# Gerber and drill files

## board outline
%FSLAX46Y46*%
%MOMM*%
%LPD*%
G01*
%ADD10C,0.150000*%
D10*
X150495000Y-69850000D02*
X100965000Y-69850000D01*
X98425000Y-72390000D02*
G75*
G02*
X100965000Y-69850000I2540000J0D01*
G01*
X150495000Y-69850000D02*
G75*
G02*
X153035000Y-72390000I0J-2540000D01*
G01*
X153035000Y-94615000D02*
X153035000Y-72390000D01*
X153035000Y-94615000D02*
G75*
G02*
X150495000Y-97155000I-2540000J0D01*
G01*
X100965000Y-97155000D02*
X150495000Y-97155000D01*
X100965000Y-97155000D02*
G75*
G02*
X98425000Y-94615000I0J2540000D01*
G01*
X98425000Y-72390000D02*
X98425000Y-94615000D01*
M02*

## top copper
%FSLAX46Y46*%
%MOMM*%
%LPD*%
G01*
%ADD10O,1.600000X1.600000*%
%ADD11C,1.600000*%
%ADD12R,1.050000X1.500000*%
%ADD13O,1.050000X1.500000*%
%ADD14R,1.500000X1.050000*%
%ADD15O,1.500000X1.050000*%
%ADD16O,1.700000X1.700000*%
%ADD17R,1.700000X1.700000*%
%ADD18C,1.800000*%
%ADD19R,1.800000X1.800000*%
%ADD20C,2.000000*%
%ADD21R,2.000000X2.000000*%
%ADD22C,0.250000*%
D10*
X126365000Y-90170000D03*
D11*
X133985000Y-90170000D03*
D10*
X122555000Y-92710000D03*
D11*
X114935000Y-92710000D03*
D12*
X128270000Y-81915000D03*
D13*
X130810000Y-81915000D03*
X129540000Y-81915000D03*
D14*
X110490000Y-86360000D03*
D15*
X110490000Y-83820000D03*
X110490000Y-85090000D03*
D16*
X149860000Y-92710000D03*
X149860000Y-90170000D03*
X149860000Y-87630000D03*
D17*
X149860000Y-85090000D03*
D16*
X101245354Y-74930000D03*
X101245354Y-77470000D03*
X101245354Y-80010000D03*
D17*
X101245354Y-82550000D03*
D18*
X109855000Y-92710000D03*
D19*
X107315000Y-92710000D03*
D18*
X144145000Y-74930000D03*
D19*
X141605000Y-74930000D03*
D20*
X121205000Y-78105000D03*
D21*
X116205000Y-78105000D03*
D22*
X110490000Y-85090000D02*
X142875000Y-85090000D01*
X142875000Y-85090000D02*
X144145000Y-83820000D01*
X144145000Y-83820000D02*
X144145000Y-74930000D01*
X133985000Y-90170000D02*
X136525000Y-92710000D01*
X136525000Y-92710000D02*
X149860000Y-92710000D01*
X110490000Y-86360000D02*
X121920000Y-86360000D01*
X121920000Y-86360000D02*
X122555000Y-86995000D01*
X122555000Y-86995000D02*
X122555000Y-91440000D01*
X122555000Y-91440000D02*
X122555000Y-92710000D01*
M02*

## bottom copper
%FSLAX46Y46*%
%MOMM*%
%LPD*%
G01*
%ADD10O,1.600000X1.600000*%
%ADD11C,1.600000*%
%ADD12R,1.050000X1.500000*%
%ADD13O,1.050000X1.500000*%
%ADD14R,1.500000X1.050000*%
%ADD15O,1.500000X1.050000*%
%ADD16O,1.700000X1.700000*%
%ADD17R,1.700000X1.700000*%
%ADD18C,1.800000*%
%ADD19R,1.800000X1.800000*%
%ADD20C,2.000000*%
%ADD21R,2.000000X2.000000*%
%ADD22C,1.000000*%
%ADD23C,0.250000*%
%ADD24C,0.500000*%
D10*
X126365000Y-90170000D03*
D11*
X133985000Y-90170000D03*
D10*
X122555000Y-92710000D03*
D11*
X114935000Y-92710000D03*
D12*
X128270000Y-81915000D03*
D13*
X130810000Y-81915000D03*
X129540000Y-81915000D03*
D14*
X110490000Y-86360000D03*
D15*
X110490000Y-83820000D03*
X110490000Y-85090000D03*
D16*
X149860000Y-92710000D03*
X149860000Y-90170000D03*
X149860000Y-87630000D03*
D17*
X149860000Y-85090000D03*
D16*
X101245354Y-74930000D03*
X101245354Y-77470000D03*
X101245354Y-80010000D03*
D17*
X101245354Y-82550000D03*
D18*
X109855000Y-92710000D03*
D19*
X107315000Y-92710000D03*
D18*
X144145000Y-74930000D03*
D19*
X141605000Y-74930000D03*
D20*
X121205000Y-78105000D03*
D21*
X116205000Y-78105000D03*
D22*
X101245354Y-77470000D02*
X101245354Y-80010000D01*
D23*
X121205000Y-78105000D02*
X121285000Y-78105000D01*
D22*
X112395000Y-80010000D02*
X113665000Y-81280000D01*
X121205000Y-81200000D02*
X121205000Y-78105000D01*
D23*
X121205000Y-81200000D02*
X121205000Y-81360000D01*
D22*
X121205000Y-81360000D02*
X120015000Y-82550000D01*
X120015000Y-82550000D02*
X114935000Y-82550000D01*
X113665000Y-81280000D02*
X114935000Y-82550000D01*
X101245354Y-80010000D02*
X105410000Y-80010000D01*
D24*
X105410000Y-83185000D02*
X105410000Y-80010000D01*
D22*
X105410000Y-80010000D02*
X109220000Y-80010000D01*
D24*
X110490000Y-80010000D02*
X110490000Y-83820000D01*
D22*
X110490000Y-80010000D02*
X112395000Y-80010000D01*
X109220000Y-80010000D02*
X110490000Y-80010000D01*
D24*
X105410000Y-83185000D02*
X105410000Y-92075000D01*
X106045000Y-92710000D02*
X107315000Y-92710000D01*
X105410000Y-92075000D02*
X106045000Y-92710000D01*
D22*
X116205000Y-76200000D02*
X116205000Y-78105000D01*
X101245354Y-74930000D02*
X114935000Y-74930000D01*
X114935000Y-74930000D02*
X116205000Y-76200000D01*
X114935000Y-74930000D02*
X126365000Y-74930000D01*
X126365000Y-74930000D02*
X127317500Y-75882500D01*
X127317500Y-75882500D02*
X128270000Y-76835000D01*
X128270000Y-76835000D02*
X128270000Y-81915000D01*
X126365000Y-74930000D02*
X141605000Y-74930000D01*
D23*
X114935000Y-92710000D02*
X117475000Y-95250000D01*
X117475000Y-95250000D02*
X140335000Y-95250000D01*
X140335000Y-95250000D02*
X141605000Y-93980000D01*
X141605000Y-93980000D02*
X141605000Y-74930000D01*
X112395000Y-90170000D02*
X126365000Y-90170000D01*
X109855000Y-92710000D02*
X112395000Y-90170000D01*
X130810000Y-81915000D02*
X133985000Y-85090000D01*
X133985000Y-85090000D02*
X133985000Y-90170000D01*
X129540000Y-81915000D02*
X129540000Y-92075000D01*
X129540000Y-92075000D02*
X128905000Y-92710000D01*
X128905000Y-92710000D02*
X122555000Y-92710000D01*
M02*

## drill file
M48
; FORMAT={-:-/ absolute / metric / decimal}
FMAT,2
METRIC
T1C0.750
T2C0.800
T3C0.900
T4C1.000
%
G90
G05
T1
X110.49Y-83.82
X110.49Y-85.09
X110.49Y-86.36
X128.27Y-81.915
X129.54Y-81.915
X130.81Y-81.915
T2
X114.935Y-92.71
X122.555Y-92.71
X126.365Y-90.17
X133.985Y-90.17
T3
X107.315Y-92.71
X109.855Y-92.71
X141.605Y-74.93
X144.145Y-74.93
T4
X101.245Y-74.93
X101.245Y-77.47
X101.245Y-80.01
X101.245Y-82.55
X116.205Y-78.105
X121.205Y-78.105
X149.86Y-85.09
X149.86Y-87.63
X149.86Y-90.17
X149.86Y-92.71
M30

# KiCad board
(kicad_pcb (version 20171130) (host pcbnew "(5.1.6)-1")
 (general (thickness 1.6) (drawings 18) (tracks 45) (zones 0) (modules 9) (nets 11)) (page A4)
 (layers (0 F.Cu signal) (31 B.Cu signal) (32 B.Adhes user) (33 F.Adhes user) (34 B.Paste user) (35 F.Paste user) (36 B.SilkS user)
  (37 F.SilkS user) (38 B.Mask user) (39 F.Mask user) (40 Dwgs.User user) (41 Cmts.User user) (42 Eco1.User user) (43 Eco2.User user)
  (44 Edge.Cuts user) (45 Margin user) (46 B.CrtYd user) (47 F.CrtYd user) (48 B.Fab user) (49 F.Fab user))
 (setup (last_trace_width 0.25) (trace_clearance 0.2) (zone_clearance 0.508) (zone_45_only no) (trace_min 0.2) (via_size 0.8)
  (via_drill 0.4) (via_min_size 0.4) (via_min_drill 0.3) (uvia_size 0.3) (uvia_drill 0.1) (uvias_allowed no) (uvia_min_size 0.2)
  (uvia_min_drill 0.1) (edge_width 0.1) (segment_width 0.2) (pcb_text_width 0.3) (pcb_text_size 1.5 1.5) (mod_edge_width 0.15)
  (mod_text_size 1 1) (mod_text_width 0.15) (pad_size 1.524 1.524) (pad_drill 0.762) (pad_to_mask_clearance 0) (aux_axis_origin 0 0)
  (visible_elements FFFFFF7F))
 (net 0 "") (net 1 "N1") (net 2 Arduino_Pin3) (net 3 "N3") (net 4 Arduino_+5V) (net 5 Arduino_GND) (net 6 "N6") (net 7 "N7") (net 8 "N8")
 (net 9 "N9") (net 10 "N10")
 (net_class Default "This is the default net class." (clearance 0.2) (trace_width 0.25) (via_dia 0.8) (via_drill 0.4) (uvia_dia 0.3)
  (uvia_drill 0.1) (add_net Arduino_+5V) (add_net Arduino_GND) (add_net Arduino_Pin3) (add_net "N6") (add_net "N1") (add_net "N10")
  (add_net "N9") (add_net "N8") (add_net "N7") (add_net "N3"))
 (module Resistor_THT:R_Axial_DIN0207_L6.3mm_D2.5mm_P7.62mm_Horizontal (layer F.Cu) (at 133.985 90.17 180)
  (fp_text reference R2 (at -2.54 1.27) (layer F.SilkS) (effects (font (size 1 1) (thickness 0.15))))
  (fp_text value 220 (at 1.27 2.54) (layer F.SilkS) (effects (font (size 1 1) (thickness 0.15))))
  (pad 2 thru_hole oval (at 7.62 0 180) (size 1.6 1.6) (drill 0.8) (layers *.Cu *.Mask) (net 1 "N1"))
  (pad 1 thru_hole circle (at 0 0 180) (size 1.6 1.6) (drill 0.8) (layers *.Cu *.Mask) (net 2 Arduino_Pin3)))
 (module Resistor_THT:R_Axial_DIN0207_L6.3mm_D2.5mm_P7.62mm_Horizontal (layer F.Cu) (at 114.935 92.71)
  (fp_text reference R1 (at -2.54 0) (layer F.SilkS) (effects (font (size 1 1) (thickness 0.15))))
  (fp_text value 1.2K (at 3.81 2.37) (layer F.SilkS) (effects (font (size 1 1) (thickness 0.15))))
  (pad 2 thru_hole oval (at 7.62 0) (size 1.6 1.6) (drill 0.8) (layers *.Cu *.Mask) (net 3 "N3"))
  (pad 1 thru_hole circle (at 0 0) (size 1.6 1.6) (drill 0.8) (layers *.Cu *.Mask) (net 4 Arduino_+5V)))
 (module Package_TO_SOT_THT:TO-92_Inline (layer F.Cu) (at 128.27 81.915)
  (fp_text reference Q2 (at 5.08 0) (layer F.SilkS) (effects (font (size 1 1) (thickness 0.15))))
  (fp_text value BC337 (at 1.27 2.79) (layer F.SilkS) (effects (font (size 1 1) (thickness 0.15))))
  (pad 1 thru_hole rect (at 0 0) (size 1.05 1.5) (drill 0.75) (layers *.Cu *.Mask) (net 4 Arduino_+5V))
  (pad 3 thru_hole oval (at 2.54 0) (size 1.05 1.5) (drill 0.75) (layers *.Cu *.Mask) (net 2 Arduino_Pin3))
  (pad 2 thru_hole oval (at 1.27 0) (size 1.05 1.5) (drill 0.75) (layers *.Cu *.Mask) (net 3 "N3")))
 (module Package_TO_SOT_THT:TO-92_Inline (layer F.Cu) (at 110.49 86.36 90)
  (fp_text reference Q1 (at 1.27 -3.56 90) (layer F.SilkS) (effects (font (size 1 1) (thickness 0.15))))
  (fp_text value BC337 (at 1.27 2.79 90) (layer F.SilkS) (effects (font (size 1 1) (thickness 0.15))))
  (pad 1 thru_hole rect (at 0 0 90) (size 1.05 1.5) (drill 0.75) (layers *.Cu *.Mask) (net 3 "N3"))
  (pad 3 thru_hole oval (at 2.54 0 90) (size 1.05 1.5) (drill 0.75) (layers *.Cu *.Mask) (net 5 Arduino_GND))
  (pad 2 thru_hole oval (at 1.27 0 90) (size 1.05 1.5) (drill 0.75) (layers *.Cu *.Mask) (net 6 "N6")))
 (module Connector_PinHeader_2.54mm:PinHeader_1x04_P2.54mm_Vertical (layer F.Cu) (at 149.86 85.09)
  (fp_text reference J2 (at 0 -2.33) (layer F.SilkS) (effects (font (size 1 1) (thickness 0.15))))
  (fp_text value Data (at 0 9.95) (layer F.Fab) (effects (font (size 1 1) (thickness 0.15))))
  (pad 4 thru_hole oval (at 0 7.62) (size 1.7 1.7) (drill 1) (layers *.Cu *.Mask) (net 2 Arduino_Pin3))
  (pad 3 thru_hole oval (at 0 5.08) (size 1.7 1.7) (drill 1) (layers *.Cu *.Mask) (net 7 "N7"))
  (pad 2 thru_hole oval (at 0 2.54) (size 1.7 1.7) (drill 1) (layers *.Cu *.Mask) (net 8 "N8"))
  (pad 1 thru_hole rect (at 0 0) (size 1.7 1.7) (drill 1) (layers *.Cu *.Mask) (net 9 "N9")))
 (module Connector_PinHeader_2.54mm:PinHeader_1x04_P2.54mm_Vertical (layer F.Cu) (at 101.245354 82.55 180)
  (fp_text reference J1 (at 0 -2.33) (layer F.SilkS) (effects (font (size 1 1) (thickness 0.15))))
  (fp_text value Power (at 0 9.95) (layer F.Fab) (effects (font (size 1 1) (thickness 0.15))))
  (pad 4 thru_hole oval (at 0 7.62 180) (size 1.7 1.7) (drill 1) (layers *.Cu *.Mask) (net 4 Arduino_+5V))
  (pad 3 thru_hole oval (at 0 5.08 180) (size 1.7 1.7) (drill 1) (layers *.Cu *.Mask) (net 5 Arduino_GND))
  (pad 2 thru_hole oval (at 0 2.54 180) (size 1.7 1.7) (drill 1) (layers *.Cu *.Mask) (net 5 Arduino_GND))
  (pad 1 thru_hole rect (at 0 0 180) (size 1.7 1.7) (drill 1) (layers *.Cu *.Mask) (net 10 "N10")))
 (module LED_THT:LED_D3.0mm (layer F.Cu) (at 107.315 92.71)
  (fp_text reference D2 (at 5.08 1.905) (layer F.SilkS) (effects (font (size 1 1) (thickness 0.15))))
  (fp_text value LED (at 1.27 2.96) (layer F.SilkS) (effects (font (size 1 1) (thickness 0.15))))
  (pad 2 thru_hole circle (at 2.54 0) (size 1.8 1.8) (drill 0.9) (layers *.Cu *.Mask) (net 1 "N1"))
  (pad 1 thru_hole rect (at 0 0) (size 1.8 1.8) (drill 0.9) (layers *.Cu *.Mask) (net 5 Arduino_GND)))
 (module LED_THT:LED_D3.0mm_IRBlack (layer F.Cu) (at 141.605 74.93)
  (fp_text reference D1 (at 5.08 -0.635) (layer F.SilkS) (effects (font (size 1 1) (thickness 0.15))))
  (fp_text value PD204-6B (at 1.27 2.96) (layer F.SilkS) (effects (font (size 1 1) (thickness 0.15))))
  (pad 2 thru_hole circle (at 2.54 0) (size 1.8 1.8) (drill 0.9) (layers *.Cu *.Mask) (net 6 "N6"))
  (pad 1 thru_hole rect (at 0 0) (size 1.8 1.8) (drill 0.9) (layers *.Cu *.Mask) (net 4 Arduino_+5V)))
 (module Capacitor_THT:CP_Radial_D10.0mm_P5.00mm (layer F.Cu) (at 116.205 78.105)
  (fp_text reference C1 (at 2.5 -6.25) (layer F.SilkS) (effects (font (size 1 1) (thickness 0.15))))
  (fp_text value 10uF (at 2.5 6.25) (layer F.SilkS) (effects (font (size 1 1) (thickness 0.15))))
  (pad 2 thru_hole circle (at 5 0) (size 2 2) (drill 1) (layers *.Cu *.Mask) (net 5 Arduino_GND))
  (pad 1 thru_hole rect (at 0 0) (size 2 2) (drill 1) (layers *.Cu *.Mask) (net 4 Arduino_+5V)))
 (gr_line (start 150.495 69.85) (end 100.965 69.85) (layer Edge.Cuts) (width 0.15))
 (gr_arc (start 100.965 72.39) (end 100.965 69.85) (angle -90) (layer Edge.Cuts) (width 0.15))
 (gr_arc (start 150.495 72.39) (end 153.035 72.39) (angle -90) (layer Edge.Cuts) (width 0.15))
 (gr_line (start 153.035 94.615) (end 153.035 72.39) (layer Edge.Cuts) (width 0.15))
 (gr_arc (start 150.495 94.615) (end 150.495 97.155) (angle -90) (layer Edge.Cuts) (width 0.15))
 (gr_line (start 100.965 97.155) (end 150.495 97.155) (layer Edge.Cuts) (width 0.15))
 (gr_arc (start 100.965 94.615) (end 98.425 94.615) (angle -90) (layer Edge.Cuts) (width 0.15))
 (gr_line (start 98.425 72.39) (end 98.425 94.615) (layer Edge.Cuts) (width 0.15))
 (segment (start 101.245354 77.47) (end 101.245354 80.01) (width 1) (layer B.Cu) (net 5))
 (segment (start 121.205 78.105) (end 121.285 78.105) (width 0.25) (layer B.Cu) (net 5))
 (segment (start 112.395 80.01) (end 113.665 81.28) (width 1) (layer B.Cu) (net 5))
 (segment (start 121.205 81.2) (end 121.205 78.105) (width 1) (layer B.Cu) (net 5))
 (segment (start 121.205 81.2) (end 121.205 81.36) (width 0.25) (layer B.Cu) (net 5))
 (segment (start 121.205 81.36) (end 120.015 82.55) (width 1) (layer B.Cu) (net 5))
 (segment (start 120.015 82.55) (end 114.935 82.55) (width 1) (layer B.Cu) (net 5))
 (segment (start 113.665 81.28) (end 114.935 82.55) (width 1) (layer B.Cu) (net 5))
 (segment (start 101.245354 80.01) (end 105.41 80.01) (width 1) (layer B.Cu) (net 5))
 (segment (start 105.41 83.185) (end 105.41 80.01) (width 0.5) (layer B.Cu) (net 5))
 (segment (start 105.41 80.01) (end 109.22 80.01) (width 1) (layer B.Cu) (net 5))
 (segment (start 110.49 80.01) (end 110.49 83.82) (width 0.5) (layer B.Cu) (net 5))
 (segment (start 110.49 80.01) (end 112.395 80.01) (width 1) (layer B.Cu) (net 5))
 (segment (start 109.22 80.01) (end 110.49 80.01) (width 1) (layer B.Cu) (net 5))
 (segment (start 105.41 83.185) (end 105.41 92.075) (width 0.5) (layer B.Cu) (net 5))
 (segment (start 106.045 92.71) (end 107.315 92.71) (width 0.5) (layer B.Cu) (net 5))
 (segment (start 105.41 92.075) (end 106.045 92.71) (width 0.5) (layer B.Cu) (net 5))
 (segment (start 116.205 76.2) (end 116.205 78.105) (width 1) (layer B.Cu) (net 4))
 (segment (start 101.245354 74.93) (end 114.935 74.93) (width 1) (layer B.Cu) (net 4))
 (segment (start 114.935 74.93) (end 116.205 76.2) (width 1) (layer B.Cu) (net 4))
 (segment (start 114.935 74.93) (end 126.365 74.93) (width 1) (layer B.Cu) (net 4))
 (segment (start 126.365 74.93) (end 127.3175 75.8825) (width 1) (layer B.Cu) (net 4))
 (segment (start 127.3175 75.8825) (end 128.27 76.835) (width 1) (layer B.Cu) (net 4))
 (segment (start 128.27 76.835) (end 128.27 81.915) (width 1) (layer B.Cu) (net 4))
 (segment (start 126.365 74.93) (end 141.605 74.93) (width 1) (layer B.Cu) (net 4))
 (segment (start 114.935 92.71) (end 117.475 95.25) (width 0.25) (layer B.Cu) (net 4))
 (segment (start 117.475 95.25) (end 140.335 95.25) (width 0.25) (layer B.Cu) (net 4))
 (segment (start 140.335 95.25) (end 141.605 93.98) (width 0.25) (layer B.Cu) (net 4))
 (segment (start 141.605 93.98) (end 141.605 74.93) (width 0.25) (layer B.Cu) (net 4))
 (segment (start 110.49 85.09) (end 142.875 85.09) (width 0.25) (layer F.Cu) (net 6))
 (segment (start 142.875 85.09) (end 144.145 83.82) (width 0.25) (layer F.Cu) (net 6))
 (segment (start 144.145 83.82) (end 144.145 74.93) (width 0.25) (layer F.Cu) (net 6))
 (segment (start 112.395 90.17) (end 126.365 90.17) (width 0.25) (layer B.Cu) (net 1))
 (segment (start 109.855 92.71) (end 112.395 90.17) (width 0.25) (layer B.Cu) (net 1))
 (segment (start 130.81 81.915) (end 133.985 85.09) (width 0.25) (layer B.Cu) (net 2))
 (segment (start 133.985 85.09) (end 133.985 90.17) (width 0.25) (layer B.Cu) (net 2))
 (segment (start 133.985 90.17) (end 136.525 92.71) (width 0.25) (layer F.Cu) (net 2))
 (segment (start 136.525 92.71) (end 149.86 92.71) (width 0.25) (layer F.Cu) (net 2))
 (segment (start 129.54 81.915) (end 129.54 92.075) (width 0.25) (layer B.Cu) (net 3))
 (segment (start 129.54 92.075) (end 128.905 92.71) (width 0.25) (layer B.Cu) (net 3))
 (segment (start 128.905 92.71) (end 122.555 92.71) (width 0.25) (layer B.Cu) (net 3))
 (segment (start 110.49 86.36) (end 121.92 86.36) (width 0.25) (layer F.Cu) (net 3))
 (segment (start 121.92 86.36) (end 122.555 86.995) (width 0.25) (layer F.Cu) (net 3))
 (segment (start 122.555 86.995) (end 122.555 91.44) (width 0.25) (layer F.Cu) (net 3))
 (segment (start 122.555 91.44) (end 122.555 92.71) (width 0.25) (layer F.Cu) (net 3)))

